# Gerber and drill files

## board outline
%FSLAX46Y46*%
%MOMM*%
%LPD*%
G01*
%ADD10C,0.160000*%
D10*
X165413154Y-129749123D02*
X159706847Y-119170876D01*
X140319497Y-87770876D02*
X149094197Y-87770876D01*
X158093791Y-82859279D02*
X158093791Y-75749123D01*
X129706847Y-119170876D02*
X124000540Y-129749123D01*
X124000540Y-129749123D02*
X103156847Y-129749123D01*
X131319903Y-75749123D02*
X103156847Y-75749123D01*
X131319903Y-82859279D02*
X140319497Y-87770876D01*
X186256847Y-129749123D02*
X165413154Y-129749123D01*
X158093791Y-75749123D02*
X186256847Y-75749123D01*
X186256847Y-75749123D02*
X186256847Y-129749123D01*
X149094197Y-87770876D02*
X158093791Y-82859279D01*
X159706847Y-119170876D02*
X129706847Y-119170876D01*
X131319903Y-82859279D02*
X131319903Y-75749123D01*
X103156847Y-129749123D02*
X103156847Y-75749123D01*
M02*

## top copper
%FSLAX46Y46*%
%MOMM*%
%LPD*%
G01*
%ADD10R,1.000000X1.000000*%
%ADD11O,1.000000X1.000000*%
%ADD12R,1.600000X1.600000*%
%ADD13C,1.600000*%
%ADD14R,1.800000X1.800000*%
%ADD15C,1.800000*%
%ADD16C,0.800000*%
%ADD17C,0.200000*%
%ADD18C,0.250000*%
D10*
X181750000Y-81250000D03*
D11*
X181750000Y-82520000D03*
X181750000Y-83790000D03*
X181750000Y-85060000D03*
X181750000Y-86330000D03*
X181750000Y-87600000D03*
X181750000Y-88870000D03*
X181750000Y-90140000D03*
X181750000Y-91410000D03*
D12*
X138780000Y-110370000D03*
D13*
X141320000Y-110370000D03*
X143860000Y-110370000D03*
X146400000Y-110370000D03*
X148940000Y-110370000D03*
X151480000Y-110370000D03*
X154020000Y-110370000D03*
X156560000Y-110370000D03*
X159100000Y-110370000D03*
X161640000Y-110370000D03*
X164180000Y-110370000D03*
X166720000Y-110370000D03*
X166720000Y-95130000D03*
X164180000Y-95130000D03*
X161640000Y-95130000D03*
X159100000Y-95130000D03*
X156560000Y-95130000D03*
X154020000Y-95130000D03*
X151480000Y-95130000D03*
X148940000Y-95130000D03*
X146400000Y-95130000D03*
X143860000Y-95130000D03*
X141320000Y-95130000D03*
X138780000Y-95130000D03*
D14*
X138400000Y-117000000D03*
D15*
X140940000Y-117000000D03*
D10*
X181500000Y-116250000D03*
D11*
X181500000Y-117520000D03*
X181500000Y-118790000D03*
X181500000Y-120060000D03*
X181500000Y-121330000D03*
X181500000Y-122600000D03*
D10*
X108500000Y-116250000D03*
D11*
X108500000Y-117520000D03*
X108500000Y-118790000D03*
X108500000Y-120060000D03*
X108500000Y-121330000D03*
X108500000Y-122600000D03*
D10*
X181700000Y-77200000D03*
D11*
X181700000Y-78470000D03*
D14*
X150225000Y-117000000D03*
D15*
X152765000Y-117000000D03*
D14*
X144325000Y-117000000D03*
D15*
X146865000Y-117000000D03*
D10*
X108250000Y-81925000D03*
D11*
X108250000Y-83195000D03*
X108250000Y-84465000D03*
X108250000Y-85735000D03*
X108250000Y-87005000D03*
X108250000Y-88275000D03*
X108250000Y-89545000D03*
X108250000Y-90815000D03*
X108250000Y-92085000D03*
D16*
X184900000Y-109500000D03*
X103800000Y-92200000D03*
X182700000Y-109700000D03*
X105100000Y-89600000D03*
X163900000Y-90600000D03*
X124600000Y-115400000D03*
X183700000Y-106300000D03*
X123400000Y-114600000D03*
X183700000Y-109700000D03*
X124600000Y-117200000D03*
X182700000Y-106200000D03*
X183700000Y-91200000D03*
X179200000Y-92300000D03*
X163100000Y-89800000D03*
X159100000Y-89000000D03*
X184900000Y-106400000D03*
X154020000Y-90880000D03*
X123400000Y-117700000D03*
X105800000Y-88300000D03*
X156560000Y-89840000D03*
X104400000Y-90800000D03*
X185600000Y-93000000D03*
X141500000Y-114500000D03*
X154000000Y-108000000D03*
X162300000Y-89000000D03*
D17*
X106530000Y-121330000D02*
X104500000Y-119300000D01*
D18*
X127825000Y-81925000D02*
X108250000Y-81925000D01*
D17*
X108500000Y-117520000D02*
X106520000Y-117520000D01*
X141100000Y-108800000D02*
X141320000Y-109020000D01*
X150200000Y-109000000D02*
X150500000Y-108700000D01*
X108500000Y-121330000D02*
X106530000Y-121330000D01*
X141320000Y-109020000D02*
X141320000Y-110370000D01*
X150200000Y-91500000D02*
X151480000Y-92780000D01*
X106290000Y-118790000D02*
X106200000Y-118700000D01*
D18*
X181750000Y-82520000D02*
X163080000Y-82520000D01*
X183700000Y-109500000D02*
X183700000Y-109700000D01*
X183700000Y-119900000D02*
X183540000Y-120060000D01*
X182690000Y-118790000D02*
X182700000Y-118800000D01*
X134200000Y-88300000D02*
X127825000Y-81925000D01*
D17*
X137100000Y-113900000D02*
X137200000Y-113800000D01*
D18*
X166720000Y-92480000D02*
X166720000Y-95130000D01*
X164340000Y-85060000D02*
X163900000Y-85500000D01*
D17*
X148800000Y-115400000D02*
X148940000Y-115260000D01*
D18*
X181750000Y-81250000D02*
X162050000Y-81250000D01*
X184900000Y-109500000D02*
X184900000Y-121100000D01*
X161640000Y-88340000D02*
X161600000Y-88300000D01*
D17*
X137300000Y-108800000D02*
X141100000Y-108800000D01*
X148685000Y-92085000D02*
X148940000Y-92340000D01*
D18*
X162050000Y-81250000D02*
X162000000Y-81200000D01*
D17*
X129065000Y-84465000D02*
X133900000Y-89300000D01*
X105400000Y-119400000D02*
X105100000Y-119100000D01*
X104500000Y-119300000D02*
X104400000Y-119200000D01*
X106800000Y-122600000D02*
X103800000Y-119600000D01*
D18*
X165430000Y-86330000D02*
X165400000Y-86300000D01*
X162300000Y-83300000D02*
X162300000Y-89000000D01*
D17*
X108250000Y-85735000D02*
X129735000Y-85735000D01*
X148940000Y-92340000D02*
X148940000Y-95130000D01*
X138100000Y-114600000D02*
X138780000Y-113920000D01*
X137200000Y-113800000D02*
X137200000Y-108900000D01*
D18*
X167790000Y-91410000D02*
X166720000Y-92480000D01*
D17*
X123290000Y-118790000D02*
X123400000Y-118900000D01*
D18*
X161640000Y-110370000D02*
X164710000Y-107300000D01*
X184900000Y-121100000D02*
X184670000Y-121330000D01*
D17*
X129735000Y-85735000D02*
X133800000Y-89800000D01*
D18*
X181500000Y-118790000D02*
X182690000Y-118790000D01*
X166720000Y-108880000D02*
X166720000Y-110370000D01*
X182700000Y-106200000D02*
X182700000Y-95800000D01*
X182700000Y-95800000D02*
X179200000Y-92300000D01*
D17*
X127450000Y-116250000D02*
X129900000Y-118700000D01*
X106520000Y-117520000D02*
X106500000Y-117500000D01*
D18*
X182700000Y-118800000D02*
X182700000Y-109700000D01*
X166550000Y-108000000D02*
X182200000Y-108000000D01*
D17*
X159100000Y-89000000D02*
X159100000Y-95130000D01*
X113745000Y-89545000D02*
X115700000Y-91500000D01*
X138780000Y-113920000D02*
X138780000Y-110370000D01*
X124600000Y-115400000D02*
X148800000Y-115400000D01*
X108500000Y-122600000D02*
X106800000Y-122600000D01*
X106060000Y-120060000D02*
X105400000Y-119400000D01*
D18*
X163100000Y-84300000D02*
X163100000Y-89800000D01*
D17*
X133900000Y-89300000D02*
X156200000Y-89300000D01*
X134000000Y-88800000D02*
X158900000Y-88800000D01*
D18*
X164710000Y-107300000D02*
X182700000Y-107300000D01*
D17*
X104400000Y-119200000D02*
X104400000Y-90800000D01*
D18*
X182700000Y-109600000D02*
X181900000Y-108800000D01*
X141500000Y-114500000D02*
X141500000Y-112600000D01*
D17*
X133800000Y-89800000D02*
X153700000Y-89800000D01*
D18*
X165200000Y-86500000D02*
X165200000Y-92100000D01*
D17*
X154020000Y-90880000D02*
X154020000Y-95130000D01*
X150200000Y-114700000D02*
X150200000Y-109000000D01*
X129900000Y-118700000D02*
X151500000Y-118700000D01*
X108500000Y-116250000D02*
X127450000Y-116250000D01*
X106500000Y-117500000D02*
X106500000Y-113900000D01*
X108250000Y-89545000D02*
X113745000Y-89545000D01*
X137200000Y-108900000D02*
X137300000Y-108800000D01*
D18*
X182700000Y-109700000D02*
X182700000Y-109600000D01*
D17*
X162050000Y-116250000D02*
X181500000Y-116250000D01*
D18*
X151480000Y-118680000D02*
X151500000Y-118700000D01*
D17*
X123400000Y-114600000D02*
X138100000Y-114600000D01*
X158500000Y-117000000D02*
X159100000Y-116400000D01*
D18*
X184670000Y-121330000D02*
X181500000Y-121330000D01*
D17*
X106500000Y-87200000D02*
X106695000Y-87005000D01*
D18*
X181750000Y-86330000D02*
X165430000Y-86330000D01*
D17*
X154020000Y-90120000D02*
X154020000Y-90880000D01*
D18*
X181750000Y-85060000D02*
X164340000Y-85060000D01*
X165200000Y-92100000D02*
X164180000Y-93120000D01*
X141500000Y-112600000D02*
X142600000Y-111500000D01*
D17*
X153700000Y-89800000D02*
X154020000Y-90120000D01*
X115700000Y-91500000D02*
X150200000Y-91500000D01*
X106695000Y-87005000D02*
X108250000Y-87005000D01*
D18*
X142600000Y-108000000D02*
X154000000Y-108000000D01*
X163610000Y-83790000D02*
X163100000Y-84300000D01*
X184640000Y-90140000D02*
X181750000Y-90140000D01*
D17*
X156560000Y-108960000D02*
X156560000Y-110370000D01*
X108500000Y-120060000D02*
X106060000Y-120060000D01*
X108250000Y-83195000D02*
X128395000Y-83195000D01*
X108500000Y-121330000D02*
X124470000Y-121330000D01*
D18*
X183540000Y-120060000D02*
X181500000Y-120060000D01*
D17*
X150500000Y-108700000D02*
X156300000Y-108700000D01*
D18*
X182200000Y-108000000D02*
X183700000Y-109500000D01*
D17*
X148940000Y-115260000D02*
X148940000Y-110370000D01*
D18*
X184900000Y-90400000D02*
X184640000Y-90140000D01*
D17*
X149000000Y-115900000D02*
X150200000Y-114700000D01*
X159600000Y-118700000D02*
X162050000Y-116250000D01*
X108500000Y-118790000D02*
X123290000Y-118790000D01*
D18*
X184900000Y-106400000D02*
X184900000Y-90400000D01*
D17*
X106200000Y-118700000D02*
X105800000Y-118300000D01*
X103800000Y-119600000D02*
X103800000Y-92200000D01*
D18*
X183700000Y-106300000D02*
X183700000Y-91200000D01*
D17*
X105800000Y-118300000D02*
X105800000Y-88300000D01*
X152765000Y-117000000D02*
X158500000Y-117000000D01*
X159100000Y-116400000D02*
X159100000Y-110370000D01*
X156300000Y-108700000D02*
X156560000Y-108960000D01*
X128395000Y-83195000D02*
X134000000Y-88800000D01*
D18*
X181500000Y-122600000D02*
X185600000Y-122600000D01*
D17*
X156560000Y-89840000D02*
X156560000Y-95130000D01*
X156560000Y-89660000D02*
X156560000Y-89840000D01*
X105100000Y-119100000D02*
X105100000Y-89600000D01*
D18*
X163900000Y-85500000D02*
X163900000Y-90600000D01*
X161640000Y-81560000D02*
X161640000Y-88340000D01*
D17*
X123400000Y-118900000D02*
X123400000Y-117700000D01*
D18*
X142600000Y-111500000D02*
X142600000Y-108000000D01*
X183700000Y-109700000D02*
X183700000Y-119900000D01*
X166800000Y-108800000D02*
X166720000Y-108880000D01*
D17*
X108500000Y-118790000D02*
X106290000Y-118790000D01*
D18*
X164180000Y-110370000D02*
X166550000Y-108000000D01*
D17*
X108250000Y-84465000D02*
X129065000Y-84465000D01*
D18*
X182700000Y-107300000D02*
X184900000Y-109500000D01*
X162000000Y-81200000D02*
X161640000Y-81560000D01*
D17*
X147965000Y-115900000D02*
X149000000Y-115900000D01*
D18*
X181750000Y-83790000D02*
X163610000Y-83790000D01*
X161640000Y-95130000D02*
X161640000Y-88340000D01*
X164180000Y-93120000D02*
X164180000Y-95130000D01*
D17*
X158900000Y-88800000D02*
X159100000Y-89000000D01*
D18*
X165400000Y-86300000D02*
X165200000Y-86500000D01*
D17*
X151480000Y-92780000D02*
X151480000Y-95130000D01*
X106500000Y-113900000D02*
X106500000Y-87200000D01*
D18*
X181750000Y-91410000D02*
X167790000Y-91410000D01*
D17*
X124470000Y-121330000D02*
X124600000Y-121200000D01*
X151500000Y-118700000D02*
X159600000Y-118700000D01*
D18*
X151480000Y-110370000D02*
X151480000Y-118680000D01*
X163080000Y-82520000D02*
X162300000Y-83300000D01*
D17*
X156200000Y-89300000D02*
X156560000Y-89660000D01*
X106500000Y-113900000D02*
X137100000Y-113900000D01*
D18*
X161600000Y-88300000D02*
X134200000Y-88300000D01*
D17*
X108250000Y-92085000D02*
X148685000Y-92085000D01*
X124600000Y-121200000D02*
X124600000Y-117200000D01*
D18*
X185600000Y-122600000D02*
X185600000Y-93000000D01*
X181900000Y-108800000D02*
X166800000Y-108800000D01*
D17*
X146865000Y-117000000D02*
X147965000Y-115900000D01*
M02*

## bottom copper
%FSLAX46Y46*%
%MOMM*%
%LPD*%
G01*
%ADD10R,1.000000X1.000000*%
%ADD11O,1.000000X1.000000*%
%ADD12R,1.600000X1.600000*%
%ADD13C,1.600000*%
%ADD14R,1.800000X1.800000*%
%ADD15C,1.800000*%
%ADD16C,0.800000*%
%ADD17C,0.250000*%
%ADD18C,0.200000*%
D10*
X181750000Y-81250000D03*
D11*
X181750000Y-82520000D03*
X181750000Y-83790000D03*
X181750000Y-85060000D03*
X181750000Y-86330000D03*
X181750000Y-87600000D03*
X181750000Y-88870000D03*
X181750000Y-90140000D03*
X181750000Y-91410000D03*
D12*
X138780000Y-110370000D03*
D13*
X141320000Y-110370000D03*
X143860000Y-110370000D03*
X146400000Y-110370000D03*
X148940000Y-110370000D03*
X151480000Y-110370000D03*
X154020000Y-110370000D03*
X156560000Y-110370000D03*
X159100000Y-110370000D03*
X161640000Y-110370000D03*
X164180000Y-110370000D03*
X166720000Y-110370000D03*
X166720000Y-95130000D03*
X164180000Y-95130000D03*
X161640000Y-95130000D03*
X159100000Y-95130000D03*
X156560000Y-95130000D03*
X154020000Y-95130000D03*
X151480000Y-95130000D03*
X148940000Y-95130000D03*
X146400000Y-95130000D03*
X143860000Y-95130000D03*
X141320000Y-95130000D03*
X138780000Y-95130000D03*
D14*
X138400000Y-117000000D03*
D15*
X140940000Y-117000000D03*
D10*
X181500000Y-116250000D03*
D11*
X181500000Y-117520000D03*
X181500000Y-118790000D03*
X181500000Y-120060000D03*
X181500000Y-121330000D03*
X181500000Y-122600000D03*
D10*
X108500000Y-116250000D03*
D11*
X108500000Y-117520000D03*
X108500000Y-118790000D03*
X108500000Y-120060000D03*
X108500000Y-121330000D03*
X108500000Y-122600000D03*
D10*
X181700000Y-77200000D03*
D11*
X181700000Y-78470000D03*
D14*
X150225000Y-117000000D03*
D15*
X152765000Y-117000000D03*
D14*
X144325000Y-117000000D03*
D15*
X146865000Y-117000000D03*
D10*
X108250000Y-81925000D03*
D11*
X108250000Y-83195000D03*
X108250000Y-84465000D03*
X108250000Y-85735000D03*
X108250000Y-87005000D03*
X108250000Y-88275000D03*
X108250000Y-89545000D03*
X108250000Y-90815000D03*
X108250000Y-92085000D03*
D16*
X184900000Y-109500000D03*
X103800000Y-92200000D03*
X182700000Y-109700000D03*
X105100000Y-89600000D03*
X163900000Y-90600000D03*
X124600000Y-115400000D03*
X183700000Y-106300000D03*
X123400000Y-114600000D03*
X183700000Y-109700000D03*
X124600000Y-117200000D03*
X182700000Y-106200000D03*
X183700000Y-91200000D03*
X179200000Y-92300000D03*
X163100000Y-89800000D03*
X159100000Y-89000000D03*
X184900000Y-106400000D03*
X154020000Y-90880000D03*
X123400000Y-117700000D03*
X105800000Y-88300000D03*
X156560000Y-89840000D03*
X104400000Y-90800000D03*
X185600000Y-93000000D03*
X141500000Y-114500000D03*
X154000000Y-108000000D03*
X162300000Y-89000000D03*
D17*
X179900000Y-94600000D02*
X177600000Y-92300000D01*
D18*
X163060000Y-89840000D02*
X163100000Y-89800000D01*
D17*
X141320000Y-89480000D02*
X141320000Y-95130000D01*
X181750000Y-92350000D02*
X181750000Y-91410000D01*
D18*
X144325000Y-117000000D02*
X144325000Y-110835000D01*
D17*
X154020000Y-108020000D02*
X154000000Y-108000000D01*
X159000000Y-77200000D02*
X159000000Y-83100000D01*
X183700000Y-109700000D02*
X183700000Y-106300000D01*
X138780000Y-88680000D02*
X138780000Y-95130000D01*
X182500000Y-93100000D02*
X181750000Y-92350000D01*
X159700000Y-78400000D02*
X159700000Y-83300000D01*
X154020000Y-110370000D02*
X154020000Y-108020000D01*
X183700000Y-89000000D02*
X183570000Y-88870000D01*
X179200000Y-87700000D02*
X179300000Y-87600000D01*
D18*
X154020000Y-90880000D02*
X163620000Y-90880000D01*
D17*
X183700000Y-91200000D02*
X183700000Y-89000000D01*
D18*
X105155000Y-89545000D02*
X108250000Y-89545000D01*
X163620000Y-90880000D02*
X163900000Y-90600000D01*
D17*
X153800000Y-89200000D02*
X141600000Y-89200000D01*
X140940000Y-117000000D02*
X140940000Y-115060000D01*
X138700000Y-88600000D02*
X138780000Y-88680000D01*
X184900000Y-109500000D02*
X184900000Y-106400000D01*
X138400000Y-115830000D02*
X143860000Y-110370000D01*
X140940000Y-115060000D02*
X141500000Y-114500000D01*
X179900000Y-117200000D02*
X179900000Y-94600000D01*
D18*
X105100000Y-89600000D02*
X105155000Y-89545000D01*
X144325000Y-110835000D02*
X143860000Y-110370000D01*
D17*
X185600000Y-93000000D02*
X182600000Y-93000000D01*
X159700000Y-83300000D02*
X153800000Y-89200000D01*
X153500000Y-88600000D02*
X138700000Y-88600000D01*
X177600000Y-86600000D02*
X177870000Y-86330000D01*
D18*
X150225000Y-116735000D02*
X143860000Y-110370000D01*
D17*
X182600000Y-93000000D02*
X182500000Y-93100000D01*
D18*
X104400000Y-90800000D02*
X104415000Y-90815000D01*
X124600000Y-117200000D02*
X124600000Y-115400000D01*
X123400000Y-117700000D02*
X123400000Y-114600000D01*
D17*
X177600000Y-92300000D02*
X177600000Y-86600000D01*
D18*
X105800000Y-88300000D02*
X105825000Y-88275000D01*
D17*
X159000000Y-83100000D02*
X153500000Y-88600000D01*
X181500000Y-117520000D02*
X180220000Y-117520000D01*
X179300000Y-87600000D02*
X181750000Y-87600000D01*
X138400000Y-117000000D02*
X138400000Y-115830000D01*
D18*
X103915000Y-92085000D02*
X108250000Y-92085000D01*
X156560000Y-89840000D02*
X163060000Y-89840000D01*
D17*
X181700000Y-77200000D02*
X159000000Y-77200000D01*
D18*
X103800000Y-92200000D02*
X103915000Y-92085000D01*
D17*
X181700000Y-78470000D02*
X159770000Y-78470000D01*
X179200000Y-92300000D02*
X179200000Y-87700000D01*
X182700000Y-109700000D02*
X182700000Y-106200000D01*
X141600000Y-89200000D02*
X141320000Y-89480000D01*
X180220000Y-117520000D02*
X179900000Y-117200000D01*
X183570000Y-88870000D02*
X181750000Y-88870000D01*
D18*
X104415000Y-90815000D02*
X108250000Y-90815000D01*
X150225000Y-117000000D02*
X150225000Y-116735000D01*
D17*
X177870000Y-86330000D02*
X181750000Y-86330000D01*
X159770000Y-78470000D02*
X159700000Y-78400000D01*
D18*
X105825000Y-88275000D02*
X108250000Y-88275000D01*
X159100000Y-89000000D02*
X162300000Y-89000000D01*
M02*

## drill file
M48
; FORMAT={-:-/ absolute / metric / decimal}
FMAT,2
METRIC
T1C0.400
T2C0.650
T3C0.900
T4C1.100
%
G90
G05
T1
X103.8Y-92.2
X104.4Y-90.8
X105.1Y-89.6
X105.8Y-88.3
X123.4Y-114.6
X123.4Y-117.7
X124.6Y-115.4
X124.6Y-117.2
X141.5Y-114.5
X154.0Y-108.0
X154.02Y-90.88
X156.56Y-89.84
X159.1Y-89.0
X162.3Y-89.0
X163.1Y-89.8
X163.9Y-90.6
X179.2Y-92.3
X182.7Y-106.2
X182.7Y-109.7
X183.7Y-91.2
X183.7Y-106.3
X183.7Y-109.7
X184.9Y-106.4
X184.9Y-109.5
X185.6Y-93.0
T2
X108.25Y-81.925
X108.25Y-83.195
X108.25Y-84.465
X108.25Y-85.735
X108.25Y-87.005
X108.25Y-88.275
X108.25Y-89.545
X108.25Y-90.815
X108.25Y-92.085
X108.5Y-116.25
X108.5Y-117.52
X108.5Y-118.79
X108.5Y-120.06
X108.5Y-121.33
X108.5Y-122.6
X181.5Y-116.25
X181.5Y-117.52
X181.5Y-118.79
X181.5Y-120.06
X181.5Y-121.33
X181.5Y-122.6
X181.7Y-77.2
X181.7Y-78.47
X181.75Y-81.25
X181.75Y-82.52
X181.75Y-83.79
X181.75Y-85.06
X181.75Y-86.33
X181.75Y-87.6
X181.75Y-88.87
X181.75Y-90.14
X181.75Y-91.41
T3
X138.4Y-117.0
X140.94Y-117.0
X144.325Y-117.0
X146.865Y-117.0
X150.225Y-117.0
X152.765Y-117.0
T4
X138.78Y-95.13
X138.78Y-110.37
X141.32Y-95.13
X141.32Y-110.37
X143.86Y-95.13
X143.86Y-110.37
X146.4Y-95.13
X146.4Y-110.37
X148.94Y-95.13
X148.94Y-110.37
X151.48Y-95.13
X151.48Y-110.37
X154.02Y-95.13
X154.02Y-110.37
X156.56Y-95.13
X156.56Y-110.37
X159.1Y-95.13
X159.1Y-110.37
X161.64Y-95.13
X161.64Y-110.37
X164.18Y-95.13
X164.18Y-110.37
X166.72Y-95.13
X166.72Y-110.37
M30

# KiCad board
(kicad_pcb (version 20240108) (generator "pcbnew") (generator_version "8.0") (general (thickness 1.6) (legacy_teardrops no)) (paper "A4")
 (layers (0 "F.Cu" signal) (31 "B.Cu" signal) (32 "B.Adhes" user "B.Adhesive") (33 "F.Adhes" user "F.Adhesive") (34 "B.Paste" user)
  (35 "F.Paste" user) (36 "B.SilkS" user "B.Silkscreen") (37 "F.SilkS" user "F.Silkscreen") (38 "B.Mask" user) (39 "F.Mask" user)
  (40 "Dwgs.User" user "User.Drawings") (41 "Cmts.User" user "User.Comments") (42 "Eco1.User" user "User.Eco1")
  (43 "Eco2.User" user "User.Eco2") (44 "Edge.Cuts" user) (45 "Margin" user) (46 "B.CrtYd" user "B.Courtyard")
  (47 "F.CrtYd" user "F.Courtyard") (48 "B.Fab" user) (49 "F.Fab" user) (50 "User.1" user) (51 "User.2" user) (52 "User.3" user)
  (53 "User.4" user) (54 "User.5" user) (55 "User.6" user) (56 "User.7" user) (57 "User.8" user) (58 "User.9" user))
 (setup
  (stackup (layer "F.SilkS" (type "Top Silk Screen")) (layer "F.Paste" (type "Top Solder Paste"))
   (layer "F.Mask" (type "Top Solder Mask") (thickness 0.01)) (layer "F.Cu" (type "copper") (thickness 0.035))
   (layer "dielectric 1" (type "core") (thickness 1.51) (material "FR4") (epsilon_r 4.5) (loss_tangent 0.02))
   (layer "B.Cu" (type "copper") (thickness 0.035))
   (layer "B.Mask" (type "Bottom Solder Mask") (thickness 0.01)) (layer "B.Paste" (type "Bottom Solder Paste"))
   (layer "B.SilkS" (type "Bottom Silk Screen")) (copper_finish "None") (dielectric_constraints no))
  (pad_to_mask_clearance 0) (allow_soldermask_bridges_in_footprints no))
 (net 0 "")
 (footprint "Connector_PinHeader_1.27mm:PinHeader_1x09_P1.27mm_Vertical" (layer "F.Cu") (at 181.75 81.25)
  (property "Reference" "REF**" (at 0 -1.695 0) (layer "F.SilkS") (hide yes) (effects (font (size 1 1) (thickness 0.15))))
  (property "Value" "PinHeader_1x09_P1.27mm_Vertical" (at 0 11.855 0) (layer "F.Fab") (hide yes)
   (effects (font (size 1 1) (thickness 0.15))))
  (pad "1" thru_hole rect (at 0 0) (size 1 1) (drill 0.65) (layers "*.Cu" "*.Mask") (remove_unused_layers no))
  (pad "2" thru_hole oval (at 0 1.27) (size 1 1) (drill 0.65) (layers "*.Cu" "*.Mask") (remove_unused_layers no))
  (pad "3" thru_hole oval (at 0 2.54) (size 1 1) (drill 0.65) (layers "*.Cu" "*.Mask") (remove_unused_layers no))
  (pad "4" thru_hole oval (at 0 3.81) (size 1 1) (drill 0.65) (layers "*.Cu" "*.Mask") (remove_unused_layers no))
  (pad "5" thru_hole oval (at 0 5.08) (size 1 1) (drill 0.65) (layers "*.Cu" "*.Mask") (remove_unused_layers no))
  (pad "6" thru_hole oval (at 0 6.35) (size 1 1) (drill 0.65) (layers "*.Cu" "*.Mask") (remove_unused_layers no))
  (pad "7" thru_hole oval (at 0 7.62) (size 1 1) (drill 0.65) (layers "*.Cu" "*.Mask") (remove_unused_layers no))
  (pad "8" thru_hole oval (at 0 8.89) (size 1 1) (drill 0.65) (layers "*.Cu" "*.Mask") (remove_unused_layers no))
  (pad "9" thru_hole oval (at 0 10.16) (size 1 1) (drill 0.65) (layers "*.Cu" "*.Mask") (remove_unused_layers no)))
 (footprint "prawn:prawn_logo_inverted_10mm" (layer "F.Cu") (at 157.7 115.3)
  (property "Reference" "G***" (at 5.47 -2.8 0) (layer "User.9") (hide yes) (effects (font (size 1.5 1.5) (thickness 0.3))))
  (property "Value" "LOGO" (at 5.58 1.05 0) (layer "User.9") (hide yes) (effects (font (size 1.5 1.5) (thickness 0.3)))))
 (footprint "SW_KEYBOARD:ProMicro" (layer "F.Cu") (at 152.75 102.75)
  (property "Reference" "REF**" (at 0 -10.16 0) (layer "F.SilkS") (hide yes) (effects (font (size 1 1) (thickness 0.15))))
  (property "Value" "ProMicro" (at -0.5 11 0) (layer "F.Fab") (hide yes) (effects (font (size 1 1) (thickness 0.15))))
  (pad "1" thru_hole rect (at -13.97 7.62) (size 1.6 1.6) (drill 1.1) (layers "*.Cu" "*.Mask" "F.SilkS") (remove_unused_layers no))
  (pad "2" thru_hole circle (at -11.43 7.62) (size 1.6 1.6) (drill 1.1) (layers "*.Cu" "*.Mask" "F.SilkS") (remove_unused_layers no))
  (pad "3" thru_hole circle (at -8.89 7.62) (size 1.6 1.6) (drill 1.1) (layers "*.Cu" "*.Mask" "F.SilkS") (remove_unused_layers no))
  (pad "4" thru_hole circle (at -6.35 7.62) (size 1.6 1.6) (drill 1.1) (layers "*.Cu" "*.Mask" "F.SilkS") (remove_unused_layers no))
  (pad "5" thru_hole circle (at -3.81 7.62) (size 1.6 1.6) (drill 1.1) (layers "*.Cu" "*.Mask" "F.SilkS") (remove_unused_layers no))
  (pad "6" thru_hole circle (at -1.27 7.62) (size 1.6 1.6) (drill 1.1) (layers "*.Cu" "*.Mask" "F.SilkS") (remove_unused_layers no))
  (pad "7" thru_hole circle (at 1.27 7.62) (size 1.6 1.6) (drill 1.1) (layers "*.Cu" "*.Mask" "F.SilkS") (remove_unused_layers no))
  (pad "8" thru_hole circle (at 3.81 7.62) (size 1.6 1.6) (drill 1.1) (layers "*.Cu" "*.Mask" "F.SilkS") (remove_unused_layers no))
  (pad "9" thru_hole circle (at 6.35 7.62) (size 1.6 1.6) (drill 1.1) (layers "*.Cu" "*.Mask" "F.SilkS") (remove_unused_layers no))
  (pad "10" thru_hole circle (at 8.89 7.62) (size 1.6 1.6) (drill 1.1) (layers "*.Cu" "*.Mask" "F.SilkS") (remove_unused_layers no))
  (pad "11" thru_hole circle (at 11.43 7.62) (size 1.6 1.6) (drill 1.1) (layers "*.Cu" "*.Mask" "F.SilkS") (remove_unused_layers no))
  (pad "12" thru_hole circle (at 13.97 7.62) (size 1.6 1.6) (drill 1.1) (layers "*.Cu" "*.Mask" "F.SilkS") (remove_unused_layers no))
  (pad "13" thru_hole circle (at 13.97 -7.62) (size 1.6 1.6) (drill 1.1) (layers "*.Cu" "*.Mask" "F.SilkS") (remove_unused_layers no))
  (pad "14" thru_hole circle (at 11.43 -7.62) (size 1.6 1.6) (drill 1.1) (layers "*.Cu" "*.Mask" "F.SilkS") (remove_unused_layers no))
  (pad "15" thru_hole circle (at 8.89 -7.62) (size 1.6 1.6) (drill 1.1) (layers "*.Cu" "*.Mask" "F.SilkS") (remove_unused_layers no))
  (pad "16" thru_hole circle (at 6.35 -7.62) (size 1.6 1.6) (drill 1.1) (layers "*.Cu" "*.Mask" "F.SilkS") (remove_unused_layers no))
  (pad "17" thru_hole circle (at 3.81 -7.62) (size 1.6 1.6) (drill 1.1) (layers "*.Cu" "*.Mask" "F.SilkS") (remove_unused_layers no))
  (pad "18" thru_hole circle (at 1.27 -7.62) (size 1.6 1.6) (drill 1.1) (layers "*.Cu" "*.Mask" "F.SilkS") (remove_unused_layers no))
  (pad "19" thru_hole circle (at -1.27 -7.62) (size 1.6 1.6) (drill 1.1) (layers "*.Cu" "*.Mask" "F.SilkS") (remove_unused_layers no))
  (pad "20" thru_hole circle (at -3.81 -7.62) (size 1.6 1.6) (drill 1.1) (layers "*.Cu" "*.Mask" "F.SilkS") (remove_unused_layers no))
  (pad "21" thru_hole circle (at -6.35 -7.62) (size 1.6 1.6) (drill 1.1) (layers "*.Cu" "*.Mask" "F.SilkS") (remove_unused_layers no))
  (pad "22" thru_hole circle (at -8.89 -7.62) (size 1.6 1.6) (drill 1.1) (layers "*.Cu" "*.Mask" "F.SilkS") (remove_unused_layers no))
  (pad "23" thru_hole circle (at -11.43 -7.62) (size 1.6 1.6) (drill 1.1) (layers "*.Cu" "*.Mask" "F.SilkS") (remove_unused_layers no))
  (pad "24" thru_hole circle (at -13.97 -7.62) (size 1.6 1.6) (drill 1.1) (layers "*.Cu" "*.Mask" "F.SilkS") (remove_unused_layers no)))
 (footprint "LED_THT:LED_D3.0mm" (layer "F.Cu") (at 138.4 117)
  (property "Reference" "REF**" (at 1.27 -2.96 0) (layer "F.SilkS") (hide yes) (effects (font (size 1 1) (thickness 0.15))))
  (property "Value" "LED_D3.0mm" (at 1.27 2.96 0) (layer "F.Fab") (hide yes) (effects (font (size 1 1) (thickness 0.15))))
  (pad "1" thru_hole rect (at 0 0) (size 1.8 1.8) (drill 0.9) (layers "*.Cu" "*.Mask") (remove_unused_layers no))
  (pad "2" thru_hole circle (at 2.54 0) (size 1.8 1.8) (drill 0.9) (layers "*.Cu" "*.Mask") (remove_unused_layers no)))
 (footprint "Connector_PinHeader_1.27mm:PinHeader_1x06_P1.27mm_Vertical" (layer "F.Cu") (at 181.5 116.25)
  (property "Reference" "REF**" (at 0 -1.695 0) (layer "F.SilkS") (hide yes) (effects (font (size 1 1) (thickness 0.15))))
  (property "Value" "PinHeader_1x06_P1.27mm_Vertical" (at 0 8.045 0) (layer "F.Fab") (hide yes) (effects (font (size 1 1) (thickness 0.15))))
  (pad "1" thru_hole rect (at 0 0) (size 1 1) (drill 0.65) (layers "*.Cu" "*.Mask") (remove_unused_layers no))
  (pad "2" thru_hole oval (at 0 1.27) (size 1 1) (drill 0.65) (layers "*.Cu" "*.Mask") (remove_unused_layers no))
  (pad "3" thru_hole oval (at 0 2.54) (size 1 1) (drill 0.65) (layers "*.Cu" "*.Mask") (remove_unused_layers no))
  (pad "4" thru_hole oval (at 0 3.81) (size 1 1) (drill 0.65) (layers "*.Cu" "*.Mask") (remove_unused_layers no))
  (pad "5" thru_hole oval (at 0 5.08) (size 1 1) (drill 0.65) (layers "*.Cu" "*.Mask") (remove_unused_layers no))
  (pad "6" thru_hole oval (at 0 6.35) (size 1 1) (drill 0.65) (layers "*.Cu" "*.Mask") (remove_unused_layers no)))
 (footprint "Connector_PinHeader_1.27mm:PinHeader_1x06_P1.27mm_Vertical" (layer "F.Cu") (at 108.5 116.25)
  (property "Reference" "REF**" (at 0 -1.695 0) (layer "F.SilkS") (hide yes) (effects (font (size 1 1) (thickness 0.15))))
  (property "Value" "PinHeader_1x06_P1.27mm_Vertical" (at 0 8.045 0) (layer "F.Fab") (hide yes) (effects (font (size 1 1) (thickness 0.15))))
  (pad "1" thru_hole rect (at 0 0) (size 1 1) (drill 0.65) (layers "*.Cu" "*.Mask") (remove_unused_layers no))
  (pad "2" thru_hole oval (at 0 1.27) (size 1 1) (drill 0.65) (layers "*.Cu" "*.Mask") (remove_unused_layers no))
  (pad "3" thru_hole oval (at 0 2.54) (size 1 1) (drill 0.65) (layers "*.Cu" "*.Mask") (remove_unused_layers no))
  (pad "4" thru_hole oval (at 0 3.81) (size 1 1) (drill 0.65) (layers "*.Cu" "*.Mask") (remove_unused_layers no))
  (pad "5" thru_hole oval (at 0 5.08) (size 1 1) (drill 0.65) (layers "*.Cu" "*.Mask") (remove_unused_layers no))
  (pad "6" thru_hole oval (at 0 6.35) (size 1 1) (drill 0.65) (layers "*.Cu" "*.Mask") (remove_unused_layers no)))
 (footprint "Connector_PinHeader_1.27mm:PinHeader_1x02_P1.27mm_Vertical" (layer "F.Cu") (at 181.7 77.2)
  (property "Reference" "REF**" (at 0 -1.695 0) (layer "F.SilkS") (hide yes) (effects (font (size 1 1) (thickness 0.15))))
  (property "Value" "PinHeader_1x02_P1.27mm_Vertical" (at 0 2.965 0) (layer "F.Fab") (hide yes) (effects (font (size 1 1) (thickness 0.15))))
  (pad "1" thru_hole rect (at 0 0) (size 1 1) (drill 0.65) (layers "*.Cu" "*.Mask") (remove_unused_layers no))
  (pad "2" thru_hole oval (at 0 1.27) (size 1 1) (drill 0.65) (layers "*.Cu" "*.Mask") (remove_unused_layers no)))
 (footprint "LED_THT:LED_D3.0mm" (layer "F.Cu") (at 150.225 117)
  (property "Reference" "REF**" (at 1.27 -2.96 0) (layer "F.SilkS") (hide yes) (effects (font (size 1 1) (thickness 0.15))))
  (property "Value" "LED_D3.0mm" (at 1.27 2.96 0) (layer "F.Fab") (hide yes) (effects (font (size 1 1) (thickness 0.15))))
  (pad "1" thru_hole rect (at 0 0) (size 1.8 1.8) (drill 0.9) (layers "*.Cu" "*.Mask") (remove_unused_layers no))
  (pad "2" thru_hole circle (at 2.54 0) (size 1.8 1.8) (drill 0.9) (layers "*.Cu" "*.Mask") (remove_unused_layers no)))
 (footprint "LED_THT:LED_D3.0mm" (layer "F.Cu") (at 144.325 117)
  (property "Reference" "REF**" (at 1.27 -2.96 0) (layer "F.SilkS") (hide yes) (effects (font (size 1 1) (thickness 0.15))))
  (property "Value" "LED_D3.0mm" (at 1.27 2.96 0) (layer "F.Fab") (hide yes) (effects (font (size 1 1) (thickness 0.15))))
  (pad "1" thru_hole rect (at 0 0) (size 1.8 1.8) (drill 0.9) (layers "*.Cu" "*.Mask") (remove_unused_layers no))
  (pad "2" thru_hole circle (at 2.54 0) (size 1.8 1.8) (drill 0.9) (layers "*.Cu" "*.Mask") (remove_unused_layers no)))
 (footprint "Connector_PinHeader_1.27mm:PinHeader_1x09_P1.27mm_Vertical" (layer "F.Cu") (at 108.25 81.925)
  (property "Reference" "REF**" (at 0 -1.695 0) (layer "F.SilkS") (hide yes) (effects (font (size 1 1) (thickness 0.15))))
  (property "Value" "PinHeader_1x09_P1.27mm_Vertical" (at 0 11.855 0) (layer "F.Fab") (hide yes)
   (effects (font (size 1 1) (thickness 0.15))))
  (pad "1" thru_hole rect (at 0 0) (size 1 1) (drill 0.65) (layers "*.Cu" "*.Mask") (remove_unused_layers no))
  (pad "2" thru_hole oval (at 0 1.27) (size 1 1) (drill 0.65) (layers "*.Cu" "*.Mask") (remove_unused_layers no))
  (pad "3" thru_hole oval (at 0 2.54) (size 1 1) (drill 0.65) (layers "*.Cu" "*.Mask") (remove_unused_layers no))
  (pad "4" thru_hole oval (at 0 3.81) (size 1 1) (drill 0.65) (layers "*.Cu" "*.Mask") (remove_unused_layers no))
  (pad "5" thru_hole oval (at 0 5.08) (size 1 1) (drill 0.65) (layers "*.Cu" "*.Mask") (remove_unused_layers no))
  (pad "6" thru_hole oval (at 0 6.35) (size 1 1) (drill 0.65) (layers "*.Cu" "*.Mask") (remove_unused_layers no))
  (pad "7" thru_hole oval (at 0 7.62) (size 1 1) (drill 0.65) (layers "*.Cu" "*.Mask") (remove_unused_layers no))
  (pad "8" thru_hole oval (at 0 8.89) (size 1 1) (drill 0.65) (layers "*.Cu" "*.Mask") (remove_unused_layers no))
  (pad "9" thru_hole oval (at 0 10.16) (size 1 1) (drill 0.65) (layers "*.Cu" "*.Mask") (remove_unused_layers no)))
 (gr_line (start 165.413154 129.749123) (end 159.706847 119.170876) (stroke (width 0.16) (type solid)) (layer "Edge.Cuts"))
 (gr_line (start 140.319497 87.770876) (end 149.094197 87.770876) (stroke (width 0.16) (type solid)) (layer "Edge.Cuts"))
 (gr_line (start 158.093791 82.859279) (end 158.093791 75.749123) (stroke (width 0.16) (type solid)) (layer "Edge.Cuts"))
 (gr_line (start 129.706847 119.170876) (end 124.00054 129.749123) (stroke (width 0.16) (type solid)) (layer "Edge.Cuts"))
 (gr_line (start 124.00054 129.749123) (end 103.156847 129.749123) (stroke (width 0.16) (type solid)) (layer "Edge.Cuts"))
 (gr_line (start 131.319903 75.749123) (end 103.156847 75.749123) (stroke (width 0.16) (type solid)) (layer "Edge.Cuts"))
 (gr_line (start 131.319903 82.859279) (end 140.319497 87.770876) (stroke (width 0.16) (type solid)) (layer "Edge.Cuts"))
 (gr_line (start 186.256847 129.749123) (end 165.413154 129.749123) (stroke (width 0.16) (type solid)) (layer "Edge.Cuts"))
 (gr_line (start 158.093791 75.749123) (end 186.256847 75.749123) (stroke (width 0.16) (type solid)) (layer "Edge.Cuts"))
 (gr_line (start 186.256847 75.749123) (end 186.256847 129.749123) (stroke (width 0.16) (type solid)) (layer "Edge.Cuts"))
 (gr_line (start 149.094197 87.770876) (end 158.093791 82.859279) (stroke (width 0.16) (type solid)) (layer "Edge.Cuts"))
 (gr_line (start 159.706847 119.170876) (end 129.706847 119.170876) (stroke (width 0.16) (type solid)) (layer "Edge.Cuts"))
 (gr_line (start 131.319903 82.859279) (end 131.319903 75.749123) (stroke (width 0.16) (type solid)) (layer "Edge.Cuts"))
 (gr_line (start 103.156847 129.749123) (end 103.156847 75.749123) (stroke (width 0.16) (type solid)) (layer "Edge.Cuts"))
 (segment (start 106.53 121.33) (end 104.5 119.3) (width 0.2) (layer "F.Cu") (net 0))
 (segment (start 127.825 81.925) (end 108.25 81.925) (width 0.25) (layer "F.Cu") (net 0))
 (segment (start 108.5 117.52) (end 106.52 117.52) (width 0.2) (layer "F.Cu") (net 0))
 (segment (start 141.1 108.8) (end 141.32 109.02) (width 0.2) (layer "F.Cu") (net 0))
 (segment (start 150.2 109) (end 150.5 108.7) (width 0.2) (layer "F.Cu") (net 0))
 (segment (start 108.5 121.33) (end 106.53 121.33) (width 0.2) (layer "F.Cu") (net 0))
 (segment (start 141.32 109.02) (end 141.32 110.37) (width 0.2) (layer "F.Cu") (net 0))
 (segment (start 150.2 91.5) (end 151.48 92.78) (width 0.2) (layer "F.Cu") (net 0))
 (segment (start 106.29 118.79) (end 106.2 118.7) (width 0.2) (layer "F.Cu") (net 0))
 (segment (start 181.75 82.52) (end 163.08 82.52) (width 0.25) (layer "F.Cu") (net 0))
 (segment (start 183.7 109.5) (end 183.7 109.7) (width 0.25) (layer "F.Cu") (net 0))
 (segment (start 183.7 119.9) (end 183.54 120.06) (width 0.25) (layer "F.Cu") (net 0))
 (segment (start 182.69 118.79) (end 182.7 118.8) (width 0.25) (layer "F.Cu") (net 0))
 (segment (start 134.2 88.3) (end 127.825 81.925) (width 0.25) (layer "F.Cu") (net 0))
 (segment (start 137.1 113.9) (end 137.2 113.8) (width 0.2) (layer "F.Cu") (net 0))
 (segment (start 166.72 92.48) (end 166.72 95.13) (width 0.25) (layer "F.Cu") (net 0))
 (segment (start 164.34 85.06) (end 163.9 85.5) (width 0.25) (layer "F.Cu") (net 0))
 (segment (start 148.8 115.4) (end 148.94 115.26) (width 0.2) (layer "F.Cu") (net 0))
 (segment (start 181.75 81.25) (end 162.05 81.25) (width 0.25) (layer "F.Cu") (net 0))
 (segment (start 184.9 109.5) (end 184.9 121.1) (width 0.25) (layer "F.Cu") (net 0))
 (segment (start 161.64 88.34) (end 161.6 88.3) (width 0.25) (layer "F.Cu") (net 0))
 (segment (start 137.3 108.8) (end 141.1 108.8) (width 0.2) (layer "F.Cu") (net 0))
 (segment (start 148.685 92.085) (end 148.94 92.34) (width 0.2) (layer "F.Cu") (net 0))
 (segment (start 162.05 81.25) (end 162 81.2) (width 0.25) (layer "F.Cu") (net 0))
 (segment (start 129.065 84.465) (end 133.9 89.3) (width 0.2) (layer "F.Cu") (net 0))
 (segment (start 105.4 119.4) (end 105.1 119.1) (width 0.2) (layer "F.Cu") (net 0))
 (segment (start 104.5 119.3) (end 104.4 119.2) (width 0.2) (layer "F.Cu") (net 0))
 (segment (start 106.8 122.6) (end 103.8 119.6) (width 0.2) (layer "F.Cu") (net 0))
 (segment (start 165.43 86.33) (end 165.4 86.3) (width 0.25) (layer "F.Cu") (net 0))
 (segment (start 162.3 83.3) (end 162.3 89) (width 0.25) (layer "F.Cu") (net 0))
 (segment (start 108.25 85.735) (end 129.735 85.735) (width 0.2) (layer "F.Cu") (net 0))
 (segment (start 148.94 92.34) (end 148.94 95.13) (width 0.2) (layer "F.Cu") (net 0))
 (segment (start 138.1 114.6) (end 138.78 113.92) (width 0.2) (layer "F.Cu") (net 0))
 (segment (start 137.2 113.8) (end 137.2 108.9) (width 0.2) (layer "F.Cu") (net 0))
 (segment (start 167.79 91.41) (end 166.72 92.48) (width 0.25) (layer "F.Cu") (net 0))
 (segment (start 123.29 118.79) (end 123.4 118.9) (width 0.2) (layer "F.Cu") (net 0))
 (segment (start 161.64 110.37) (end 164.71 107.3) (width 0.25) (layer "F.Cu") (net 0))
 (segment (start 184.9 121.1) (end 184.67 121.33) (width 0.25) (layer "F.Cu") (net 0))
 (segment (start 129.735 85.735) (end 133.8 89.8) (width 0.2) (layer "F.Cu") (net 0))
 (segment (start 181.5 118.79) (end 182.69 118.79) (width 0.25) (layer "F.Cu") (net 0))
 (segment (start 166.72 108.88) (end 166.72 110.37) (width 0.25) (layer "F.Cu") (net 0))
 (segment (start 182.7 106.2) (end 182.7 95.8) (width 0.25) (layer "F.Cu") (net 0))
 (segment (start 182.7 95.8) (end 179.2 92.3) (width 0.25) (layer "F.Cu") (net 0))
 (segment (start 127.45 116.25) (end 129.9 118.7) (width 0.2) (layer "F.Cu") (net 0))
 (segment (start 106.52 117.52) (end 106.5 117.5) (width 0.2) (layer "F.Cu") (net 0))
 (segment (start 182.7 118.8) (end 182.7 109.7) (width 0.25) (layer "F.Cu") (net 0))
 (segment (start 166.55 108) (end 182.2 108) (width 0.25) (layer "F.Cu") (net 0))
 (segment (start 159.1 89) (end 159.1 95.13) (width 0.2) (layer "F.Cu") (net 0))
 (segment (start 113.745 89.545) (end 115.7 91.5) (width 0.2) (layer "F.Cu") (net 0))
 (segment (start 138.78 113.92) (end 138.78 110.37) (width 0.2) (layer "F.Cu") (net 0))
 (segment (start 124.6 115.4) (end 148.8 115.4) (width 0.2) (layer "F.Cu") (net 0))
 (segment (start 108.5 122.6) (end 106.8 122.6) (width 0.2) (layer "F.Cu") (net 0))
 (segment (start 106.06 120.06) (end 105.4 119.4) (width 0.2) (layer "F.Cu") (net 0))
 (segment (start 163.1 84.3) (end 163.1 89.8) (width 0.25) (layer "F.Cu") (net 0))
 (segment (start 133.9 89.3) (end 156.2 89.3) (width 0.2) (layer "F.Cu") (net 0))
 (segment (start 134 88.8) (end 158.9 88.8) (width 0.2) (layer "F.Cu") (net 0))
 (segment (start 164.71 107.3) (end 182.7 107.3) (width 0.25) (layer "F.Cu") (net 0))
 (segment (start 104.4 119.2) (end 104.4 90.8) (width 0.2) (layer "F.Cu") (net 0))
 (segment (start 182.7 109.6) (end 181.9 108.8) (width 0.25) (layer "F.Cu") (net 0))
 (segment (start 141.5 114.5) (end 141.5 112.6) (width 0.25) (layer "F.Cu") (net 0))
 (segment (start 133.8 89.8) (end 153.7 89.8) (width 0.2) (layer "F.Cu") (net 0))
 (segment (start 165.2 86.5) (end 165.2 92.1) (width 0.25) (layer "F.Cu") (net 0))
 (segment (start 154.02 90.88) (end 154.02 95.13) (width 0.2) (layer "F.Cu") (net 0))
 (segment (start 150.2 114.7) (end 150.2 109) (width 0.2) (layer "F.Cu") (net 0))
 (segment (start 129.9 118.7) (end 151.5 118.7) (width 0.2) (layer "F.Cu") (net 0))
 (segment (start 108.5 116.25) (end 127.45 116.25) (width 0.2) (layer "F.Cu") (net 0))
 (segment (start 106.5 117.5) (end 106.5 113.9) (width 0.2) (layer "F.Cu") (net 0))
 (segment (start 108.25 89.545) (end 113.745 89.545) (width 0.2) (layer "F.Cu") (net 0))
 (segment (start 137.2 108.9) (end 137.3 108.8) (width 0.2) (layer "F.Cu") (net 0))
 (segment (start 182.7 109.7) (end 182.7 109.6) (width 0.25) (layer "F.Cu") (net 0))
 (segment (start 162.05 116.25) (end 181.5 116.25) (width 0.2) (layer "F.Cu") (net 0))
 (segment (start 151.48 118.68) (end 151.5 118.7) (width 0.25) (layer "F.Cu") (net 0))
 (segment (start 123.4 114.6) (end 138.1 114.6) (width 0.2) (layer "F.Cu") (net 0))
 (segment (start 158.5 117) (end 159.1 116.4) (width 0.2) (layer "F.Cu") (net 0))
 (segment (start 184.67 121.33) (end 181.5 121.33) (width 0.25) (layer "F.Cu") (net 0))
 (segment (start 106.5 87.2) (end 106.695 87.005) (width 0.2) (layer "F.Cu") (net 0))
 (segment (start 181.75 86.33) (end 165.43 86.33) (width 0.25) (layer "F.Cu") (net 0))
 (segment (start 154.02 90.12) (end 154.02 90.88) (width 0.2) (layer "F.Cu") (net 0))
 (segment (start 181.75 85.06) (end 164.34 85.06) (width 0.25) (layer "F.Cu") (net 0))
 (segment (start 165.2 92.1) (end 164.18 93.12) (width 0.25) (layer "F.Cu") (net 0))
 (segment (start 141.5 112.6) (end 142.6 111.5) (width 0.25) (layer "F.Cu") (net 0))
 (segment (start 153.7 89.8) (end 154.02 90.12) (width 0.2) (layer "F.Cu") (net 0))
 (segment (start 115.7 91.5) (end 150.2 91.5) (width 0.2) (layer "F.Cu") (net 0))
 (segment (start 106.695 87.005) (end 108.25 87.005) (width 0.2) (layer "F.Cu") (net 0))
 (segment (start 142.6 108) (end 154 108) (width 0.25) (layer "F.Cu") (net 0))
 (segment (start 163.61 83.79) (end 163.1 84.3) (width 0.25) (layer "F.Cu") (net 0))
 (segment (start 184.64 90.14) (end 181.75 90.14) (width 0.25) (layer "F.Cu") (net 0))
 (segment (start 156.56 108.96) (end 156.56 110.37) (width 0.2) (layer "F.Cu") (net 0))
 (segment (start 108.5 120.06) (end 106.06 120.06) (width 0.2) (layer "F.Cu") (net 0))
 (segment (start 108.25 83.195) (end 128.395 83.195) (width 0.2) (layer "F.Cu") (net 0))
 (segment (start 108.5 121.33) (end 124.47 121.33) (width 0.2) (layer "F.Cu") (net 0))
 (segment (start 183.54 120.06) (end 181.5 120.06) (width 0.25) (layer "F.Cu") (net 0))
 (segment (start 150.5 108.7) (end 156.3 108.7) (width 0.2) (layer "F.Cu") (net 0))
 (segment (start 182.2 108) (end 183.7 109.5) (width 0.25) (layer "F.Cu") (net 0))
 (segment (start 148.94 115.26) (end 148.94 110.37) (width 0.2) (layer "F.Cu") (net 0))
 (segment (start 184.9 90.4) (end 184.64 90.14) (width 0.25) (layer "F.Cu") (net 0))
 (segment (start 149 115.9) (end 150.2 114.7) (width 0.2) (layer "F.Cu") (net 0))
 (segment (start 159.6 118.7) (end 162.05 116.25) (width 0.2) (layer "F.Cu") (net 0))
 (segment (start 108.5 118.79) (end 123.29 118.79) (width 0.2) (layer "F.Cu") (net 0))
 (segment (start 184.9 106.4) (end 184.9 90.4) (width 0.25) (layer "F.Cu") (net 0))
 (segment (start 106.2 118.7) (end 105.8 118.3) (width 0.2) (layer "F.Cu") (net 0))
 (segment (start 103.8 119.6) (end 103.8 92.2) (width 0.2) (layer "F.Cu") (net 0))
 (segment (start 183.7 106.3) (end 183.7 91.2) (width 0.25) (layer "F.Cu") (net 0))
 (segment (start 105.8 118.3) (end 105.8 88.3) (width 0.2) (layer "F.Cu") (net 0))
 (segment (start 152.765 117) (end 158.5 117) (width 0.2) (layer "F.Cu") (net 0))
 (segment (start 159.1 116.4) (end 159.1 110.37) (width 0.2) (layer "F.Cu") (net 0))
 (segment (start 156.3 108.7) (end 156.56 108.96) (width 0.2) (layer "F.Cu") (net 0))
 (segment (start 128.395 83.195) (end 134 88.8) (width 0.2) (layer "F.Cu") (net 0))
 (segment (start 181.5 122.6) (end 185.6 122.6) (width 0.25) (layer "F.Cu") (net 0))
 (segment (start 156.56 89.84) (end 156.56 95.13) (width 0.2) (layer "F.Cu") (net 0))
 (segment (start 156.56 89.66) (end 156.56 89.84) (width 0.2) (layer "F.Cu") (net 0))
 (segment (start 105.1 119.1) (end 105.1 89.6) (width 0.2) (layer "F.Cu") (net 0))
 (segment (start 163.9 85.5) (end 163.9 90.6) (width 0.25) (layer "F.Cu") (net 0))
 (segment (start 161.64 81.56) (end 161.64 88.34) (width 0.25) (layer "F.Cu") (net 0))
 (segment (start 123.4 118.9) (end 123.4 117.7) (width 0.2) (layer "F.Cu") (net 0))
 (segment (start 142.6 111.5) (end 142.6 108) (width 0.25) (layer "F.Cu") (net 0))
 (segment (start 183.7 109.7) (end 183.7 119.9) (width 0.25) (layer "F.Cu") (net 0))
 (segment (start 166.8 108.8) (end 166.72 108.88) (width 0.25) (layer "F.Cu") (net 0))
 (segment (start 108.5 118.79) (end 106.29 118.79) (width 0.2) (layer "F.Cu") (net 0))
 (segment (start 164.18 110.37) (end 166.55 108) (width 0.25) (layer "F.Cu") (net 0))
 (segment (start 108.25 84.465) (end 129.065 84.465) (width 0.2) (layer "F.Cu") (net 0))
 (segment (start 182.7 107.3) (end 184.9 109.5) (width 0.25) (layer "F.Cu") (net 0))
 (segment (start 162 81.2) (end 161.64 81.56) (width 0.25) (layer "F.Cu") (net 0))
 (segment (start 147.965 115.9) (end 149 115.9) (width 0.2) (layer "F.Cu") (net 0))
 (segment (start 181.75 83.79) (end 163.61 83.79) (width 0.25) (layer "F.Cu") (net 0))
 (segment (start 161.64 95.13) (end 161.64 88.34) (width 0.25) (layer "F.Cu") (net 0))
 (segment (start 164.18 93.12) (end 164.18 95.13) (width 0.25) (layer "F.Cu") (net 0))
 (segment (start 158.9 88.8) (end 159.1 89) (width 0.2) (layer "F.Cu") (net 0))
 (segment (start 165.4 86.3) (end 165.2 86.5) (width 0.25) (layer "F.Cu") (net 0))
 (segment (start 151.48 92.78) (end 151.48 95.13) (width 0.2) (layer "F.Cu") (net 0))
 (segment (start 106.5 113.9) (end 106.5 87.2) (width 0.2) (layer "F.Cu") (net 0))
 (segment (start 181.75 91.41) (end 167.79 91.41) (width 0.25) (layer "F.Cu") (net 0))
 (segment (start 124.47 121.33) (end 124.6 121.2) (width 0.2) (layer "F.Cu") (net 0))
 (segment (start 151.5 118.7) (end 159.6 118.7) (width 0.2) (layer "F.Cu") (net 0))
 (segment (start 151.48 110.37) (end 151.48 118.68) (width 0.25) (layer "F.Cu") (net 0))
 (segment (start 163.08 82.52) (end 162.3 83.3) (width 0.25) (layer "F.Cu") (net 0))
 (segment (start 156.2 89.3) (end 156.56 89.66) (width 0.2) (layer "F.Cu") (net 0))
 (segment (start 106.5 113.9) (end 137.1 113.9) (width 0.2) (layer "F.Cu") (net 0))
 (segment (start 161.6 88.3) (end 134.2 88.3) (width 0.25) (layer "F.Cu") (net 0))
 (segment (start 108.25 92.085) (end 148.685 92.085) (width 0.2) (layer "F.Cu") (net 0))
 (segment (start 124.6 121.2) (end 124.6 117.2) (width 0.2) (layer "F.Cu") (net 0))
 (segment (start 185.6 122.6) (end 185.6 93) (width 0.25) (layer "F.Cu") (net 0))
 (segment (start 181.9 108.8) (end 166.8 108.8) (width 0.25) (layer "F.Cu") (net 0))
 (segment (start 146.865 117) (end 147.965 115.9) (width 0.2) (layer "F.Cu") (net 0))
 (via (at 184.9 109.5) (size 0.8) (drill 0.4) (layers "F.Cu" "B.Cu") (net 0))
 (via (at 103.8 92.2) (size 0.8) (drill 0.4) (layers "F.Cu" "B.Cu") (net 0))
 (via (at 182.7 109.7) (size 0.8) (drill 0.4) (layers "F.Cu" "B.Cu") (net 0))
 (via (at 105.1 89.6) (size 0.8) (drill 0.4) (layers "F.Cu" "B.Cu") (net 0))
 (via (at 163.9 90.6) (size 0.8) (drill 0.4) (layers "F.Cu" "B.Cu") (free yes) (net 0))
 (via (at 124.6 115.4) (size 0.8) (drill 0.4) (layers "F.Cu" "B.Cu") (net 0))
 (via (at 183.7 106.3) (size 0.8) (drill 0.4) (layers "F.Cu" "B.Cu") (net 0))
 (via (at 123.4 114.6) (size 0.8) (drill 0.4) (layers "F.Cu" "B.Cu") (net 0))
 (via (at 183.7 109.7) (size 0.8) (drill 0.4) (layers "F.Cu" "B.Cu") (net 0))
 (via (at 124.6 117.2) (size 0.8) (drill 0.4) (layers "F.Cu" "B.Cu") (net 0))
 (via (at 182.7 106.2) (size 0.8) (drill 0.4) (layers "F.Cu" "B.Cu") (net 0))
 (via (at 183.7 91.2) (size 0.8) (drill 0.4) (layers "F.Cu" "B.Cu") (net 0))
 (via (at 179.2 92.3) (size 0.8) (drill 0.4) (layers "F.Cu" "B.Cu") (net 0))
 (via (at 163.1 89.8) (size 0.8) (drill 0.4) (layers "F.Cu" "B.Cu") (free yes) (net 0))
 (via (at 159.1 89) (size 0.8) (drill 0.4) (layers "F.Cu" "B.Cu") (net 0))
 (via (at 184.9 106.4) (size 0.8) (drill 0.4) (layers "F.Cu" "B.Cu") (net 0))
 (via (at 154.02 90.88) (size 0.8) (drill 0.4) (layers "F.Cu" "B.Cu") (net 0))
 (via (at 123.4 117.7) (size 0.8) (drill 0.4) (layers "F.Cu" "B.Cu") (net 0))
 (via (at 105.8 88.3) (size 0.8) (drill 0.4) (layers "F.Cu" "B.Cu") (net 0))
 (via (at 156.56 89.84) (size 0.8) (drill 0.4) (layers "F.Cu" "B.Cu") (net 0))
 (via (at 104.4 90.8) (size 0.8) (drill 0.4) (layers "F.Cu" "B.Cu") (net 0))
 (via (at 185.6 93) (size 0.8) (drill 0.4) (layers "F.Cu" "B.Cu") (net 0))
 (via (at 141.5 114.5) (size 0.8) (drill 0.4) (layers "F.Cu" "B.Cu") (free yes) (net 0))
 (via (at 154 108) (size 0.8) (drill 0.4) (layers "F.Cu" "B.Cu") (free yes) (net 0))
 (via (at 162.3 89) (size 0.8) (drill 0.4) (layers "F.Cu" "B.Cu") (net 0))
 (segment (start 179.9 94.6) (end 177.6 92.3) (width 0.25) (layer "B.Cu") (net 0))
 (segment (start 163.06 89.84) (end 163.1 89.8) (width 0.2) (layer "B.Cu") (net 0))
 (segment (start 141.32 89.48) (end 141.32 95.13) (width 0.25) (layer "B.Cu") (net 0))
 (segment (start 181.75 92.35) (end 181.75 91.41) (width 0.25) (layer "B.Cu") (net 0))
 (segment (start 144.325 117) (end 144.325 110.835) (width 0.2) (layer "B.Cu") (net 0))
 (segment (start 154.02 108.02) (end 154 108) (width 0.25) (layer "B.Cu") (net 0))
 (segment (start 159 77.2) (end 159 83.1) (width 0.25) (layer "B.Cu") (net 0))
 (segment (start 183.7 109.7) (end 183.7 106.3) (width 0.25) (layer "B.Cu") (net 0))
 (segment (start 138.78 88.68) (end 138.78 95.13) (width 0.25) (layer "B.Cu") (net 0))
 (segment (start 182.5 93.1) (end 181.75 92.35) (width 0.25) (layer "B.Cu") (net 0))
 (segment (start 159.7 78.4) (end 159.7 83.3) (width 0.25) (layer "B.Cu") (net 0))
 (segment (start 154.02 110.37) (end 154.02 108.02) (width 0.25) (layer "B.Cu") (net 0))
 (segment (start 183.7 89) (end 183.57 88.87) (width 0.25) (layer "B.Cu") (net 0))
 (segment (start 179.2 87.7) (end 179.3 87.6) (width 0.25) (layer "B.Cu") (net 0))
 (segment (start 154.02 90.88) (end 163.62 90.88) (width 0.2) (layer "B.Cu") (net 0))
 (segment (start 183.7 91.2) (end 183.7 89) (width 0.25) (layer "B.Cu") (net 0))
 (segment (start 105.155 89.545) (end 108.25 89.545) (width 0.2) (layer "B.Cu") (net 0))
 (segment (start 163.62 90.88) (end 163.9 90.6) (width 0.2) (layer "B.Cu") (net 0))
 (segment (start 153.8 89.2) (end 141.6 89.2) (width 0.25) (layer "B.Cu") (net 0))
 (segment (start 140.94 117) (end 140.94 115.06) (width 0.25) (layer "B.Cu") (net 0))
 (segment (start 138.7 88.6) (end 138.78 88.68) (width 0.25) (layer "B.Cu") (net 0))
 (segment (start 184.9 109.5) (end 184.9 106.4) (width 0.25) (layer "B.Cu") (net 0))
 (segment (start 138.4 115.83) (end 143.86 110.37) (width 0.25) (layer "B.Cu") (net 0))
 (segment (start 140.94 115.06) (end 141.5 114.5) (width 0.25) (layer "B.Cu") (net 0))
 (segment (start 179.9 117.2) (end 179.9 94.6) (width 0.25) (layer "B.Cu") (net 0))
 (segment (start 105.1 89.6) (end 105.155 89.545) (width 0.2) (layer "B.Cu") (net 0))
 (segment (start 144.325 110.835) (end 143.86 110.37) (width 0.2) (layer "B.Cu") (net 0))
 (segment (start 185.6 93) (end 182.6 93) (width 0.25) (layer "B.Cu") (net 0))
 (segment (start 159.7 83.3) (end 153.8 89.2) (width 0.25) (layer "B.Cu") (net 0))
 (segment (start 153.5 88.6) (end 138.7 88.6) (width 0.25) (layer "B.Cu") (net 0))
 (segment (start 177.6 86.6) (end 177.87 86.33) (width 0.25) (layer "B.Cu") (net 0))
 (segment (start 150.225 116.735) (end 143.86 110.37) (width 0.2) (layer "B.Cu") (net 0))
 (segment (start 182.6 93) (end 182.5 93.1) (width 0.25) (layer "B.Cu") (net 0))
 (segment (start 104.4 90.8) (end 104.415 90.815) (width 0.2) (layer "B.Cu") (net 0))
 (segment (start 124.6 117.2) (end 124.6 115.4) (width 0.2) (layer "B.Cu") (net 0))
 (segment (start 123.4 117.7) (end 123.4 114.6) (width 0.2) (layer "B.Cu") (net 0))
 (segment (start 177.6 92.3) (end 177.6 86.6) (width 0.25) (layer "B.Cu") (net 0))
 (segment (start 105.8 88.3) (end 105.825 88.275) (width 0.2) (layer "B.Cu") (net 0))
 (segment (start 159 83.1) (end 153.5 88.6) (width 0.25) (layer "B.Cu") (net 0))
 (segment (start 181.5 117.52) (end 180.22 117.52) (width 0.25) (layer "B.Cu") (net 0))
 (segment (start 179.3 87.6) (end 181.75 87.6) (width 0.25) (layer "B.Cu") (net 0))
 (segment (start 138.4 117) (end 138.4 115.83) (width 0.25) (layer "B.Cu") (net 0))
 (segment (start 103.915 92.085) (end 108.25 92.085) (width 0.2) (layer "B.Cu") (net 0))
 (segment (start 156.56 89.84) (end 163.06 89.84) (width 0.2) (layer "B.Cu") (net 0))
 (segment (start 181.7 77.2) (end 159 77.2) (width 0.25) (layer "B.Cu") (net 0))
 (segment (start 103.8 92.2) (end 103.915 92.085) (width 0.2) (layer "B.Cu") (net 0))
 (segment (start 181.7 78.47) (end 159.77 78.47) (width 0.25) (layer "B.Cu") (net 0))
 (segment (start 179.2 92.3) (end 179.2 87.7) (width 0.25) (layer "B.Cu") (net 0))
 (segment (start 182.7 109.7) (end 182.7 106.2) (width 0.25) (layer "B.Cu") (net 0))
 (segment (start 141.6 89.2) (end 141.32 89.48) (width 0.25) (layer "B.Cu") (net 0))
 (segment (start 180.22 117.52) (end 179.9 117.2) (width 0.25) (layer "B.Cu") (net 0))
 (segment (start 183.57 88.87) (end 181.75 88.87) (width 0.25) (layer "B.Cu") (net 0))
 (segment (start 104.415 90.815) (end 108.25 90.815) (width 0.2) (layer "B.Cu") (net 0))
 (segment (start 150.225 117) (end 150.225 116.735) (width 0.2) (layer "B.Cu") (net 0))
 (segment (start 177.87 86.33) (end 181.75 86.33) (width 0.25) (layer "B.Cu") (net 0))
 (segment (start 159.77 78.47) (end 159.7 78.4) (width 0.25) (layer "B.Cu") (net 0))
 (segment (start 105.825 88.275) (end 108.25 88.275) (width 0.2) (layer "B.Cu") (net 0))
 (segment (start 159.1 89) (end 162.3 89) (width 0.2) (layer "B.Cu") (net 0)))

